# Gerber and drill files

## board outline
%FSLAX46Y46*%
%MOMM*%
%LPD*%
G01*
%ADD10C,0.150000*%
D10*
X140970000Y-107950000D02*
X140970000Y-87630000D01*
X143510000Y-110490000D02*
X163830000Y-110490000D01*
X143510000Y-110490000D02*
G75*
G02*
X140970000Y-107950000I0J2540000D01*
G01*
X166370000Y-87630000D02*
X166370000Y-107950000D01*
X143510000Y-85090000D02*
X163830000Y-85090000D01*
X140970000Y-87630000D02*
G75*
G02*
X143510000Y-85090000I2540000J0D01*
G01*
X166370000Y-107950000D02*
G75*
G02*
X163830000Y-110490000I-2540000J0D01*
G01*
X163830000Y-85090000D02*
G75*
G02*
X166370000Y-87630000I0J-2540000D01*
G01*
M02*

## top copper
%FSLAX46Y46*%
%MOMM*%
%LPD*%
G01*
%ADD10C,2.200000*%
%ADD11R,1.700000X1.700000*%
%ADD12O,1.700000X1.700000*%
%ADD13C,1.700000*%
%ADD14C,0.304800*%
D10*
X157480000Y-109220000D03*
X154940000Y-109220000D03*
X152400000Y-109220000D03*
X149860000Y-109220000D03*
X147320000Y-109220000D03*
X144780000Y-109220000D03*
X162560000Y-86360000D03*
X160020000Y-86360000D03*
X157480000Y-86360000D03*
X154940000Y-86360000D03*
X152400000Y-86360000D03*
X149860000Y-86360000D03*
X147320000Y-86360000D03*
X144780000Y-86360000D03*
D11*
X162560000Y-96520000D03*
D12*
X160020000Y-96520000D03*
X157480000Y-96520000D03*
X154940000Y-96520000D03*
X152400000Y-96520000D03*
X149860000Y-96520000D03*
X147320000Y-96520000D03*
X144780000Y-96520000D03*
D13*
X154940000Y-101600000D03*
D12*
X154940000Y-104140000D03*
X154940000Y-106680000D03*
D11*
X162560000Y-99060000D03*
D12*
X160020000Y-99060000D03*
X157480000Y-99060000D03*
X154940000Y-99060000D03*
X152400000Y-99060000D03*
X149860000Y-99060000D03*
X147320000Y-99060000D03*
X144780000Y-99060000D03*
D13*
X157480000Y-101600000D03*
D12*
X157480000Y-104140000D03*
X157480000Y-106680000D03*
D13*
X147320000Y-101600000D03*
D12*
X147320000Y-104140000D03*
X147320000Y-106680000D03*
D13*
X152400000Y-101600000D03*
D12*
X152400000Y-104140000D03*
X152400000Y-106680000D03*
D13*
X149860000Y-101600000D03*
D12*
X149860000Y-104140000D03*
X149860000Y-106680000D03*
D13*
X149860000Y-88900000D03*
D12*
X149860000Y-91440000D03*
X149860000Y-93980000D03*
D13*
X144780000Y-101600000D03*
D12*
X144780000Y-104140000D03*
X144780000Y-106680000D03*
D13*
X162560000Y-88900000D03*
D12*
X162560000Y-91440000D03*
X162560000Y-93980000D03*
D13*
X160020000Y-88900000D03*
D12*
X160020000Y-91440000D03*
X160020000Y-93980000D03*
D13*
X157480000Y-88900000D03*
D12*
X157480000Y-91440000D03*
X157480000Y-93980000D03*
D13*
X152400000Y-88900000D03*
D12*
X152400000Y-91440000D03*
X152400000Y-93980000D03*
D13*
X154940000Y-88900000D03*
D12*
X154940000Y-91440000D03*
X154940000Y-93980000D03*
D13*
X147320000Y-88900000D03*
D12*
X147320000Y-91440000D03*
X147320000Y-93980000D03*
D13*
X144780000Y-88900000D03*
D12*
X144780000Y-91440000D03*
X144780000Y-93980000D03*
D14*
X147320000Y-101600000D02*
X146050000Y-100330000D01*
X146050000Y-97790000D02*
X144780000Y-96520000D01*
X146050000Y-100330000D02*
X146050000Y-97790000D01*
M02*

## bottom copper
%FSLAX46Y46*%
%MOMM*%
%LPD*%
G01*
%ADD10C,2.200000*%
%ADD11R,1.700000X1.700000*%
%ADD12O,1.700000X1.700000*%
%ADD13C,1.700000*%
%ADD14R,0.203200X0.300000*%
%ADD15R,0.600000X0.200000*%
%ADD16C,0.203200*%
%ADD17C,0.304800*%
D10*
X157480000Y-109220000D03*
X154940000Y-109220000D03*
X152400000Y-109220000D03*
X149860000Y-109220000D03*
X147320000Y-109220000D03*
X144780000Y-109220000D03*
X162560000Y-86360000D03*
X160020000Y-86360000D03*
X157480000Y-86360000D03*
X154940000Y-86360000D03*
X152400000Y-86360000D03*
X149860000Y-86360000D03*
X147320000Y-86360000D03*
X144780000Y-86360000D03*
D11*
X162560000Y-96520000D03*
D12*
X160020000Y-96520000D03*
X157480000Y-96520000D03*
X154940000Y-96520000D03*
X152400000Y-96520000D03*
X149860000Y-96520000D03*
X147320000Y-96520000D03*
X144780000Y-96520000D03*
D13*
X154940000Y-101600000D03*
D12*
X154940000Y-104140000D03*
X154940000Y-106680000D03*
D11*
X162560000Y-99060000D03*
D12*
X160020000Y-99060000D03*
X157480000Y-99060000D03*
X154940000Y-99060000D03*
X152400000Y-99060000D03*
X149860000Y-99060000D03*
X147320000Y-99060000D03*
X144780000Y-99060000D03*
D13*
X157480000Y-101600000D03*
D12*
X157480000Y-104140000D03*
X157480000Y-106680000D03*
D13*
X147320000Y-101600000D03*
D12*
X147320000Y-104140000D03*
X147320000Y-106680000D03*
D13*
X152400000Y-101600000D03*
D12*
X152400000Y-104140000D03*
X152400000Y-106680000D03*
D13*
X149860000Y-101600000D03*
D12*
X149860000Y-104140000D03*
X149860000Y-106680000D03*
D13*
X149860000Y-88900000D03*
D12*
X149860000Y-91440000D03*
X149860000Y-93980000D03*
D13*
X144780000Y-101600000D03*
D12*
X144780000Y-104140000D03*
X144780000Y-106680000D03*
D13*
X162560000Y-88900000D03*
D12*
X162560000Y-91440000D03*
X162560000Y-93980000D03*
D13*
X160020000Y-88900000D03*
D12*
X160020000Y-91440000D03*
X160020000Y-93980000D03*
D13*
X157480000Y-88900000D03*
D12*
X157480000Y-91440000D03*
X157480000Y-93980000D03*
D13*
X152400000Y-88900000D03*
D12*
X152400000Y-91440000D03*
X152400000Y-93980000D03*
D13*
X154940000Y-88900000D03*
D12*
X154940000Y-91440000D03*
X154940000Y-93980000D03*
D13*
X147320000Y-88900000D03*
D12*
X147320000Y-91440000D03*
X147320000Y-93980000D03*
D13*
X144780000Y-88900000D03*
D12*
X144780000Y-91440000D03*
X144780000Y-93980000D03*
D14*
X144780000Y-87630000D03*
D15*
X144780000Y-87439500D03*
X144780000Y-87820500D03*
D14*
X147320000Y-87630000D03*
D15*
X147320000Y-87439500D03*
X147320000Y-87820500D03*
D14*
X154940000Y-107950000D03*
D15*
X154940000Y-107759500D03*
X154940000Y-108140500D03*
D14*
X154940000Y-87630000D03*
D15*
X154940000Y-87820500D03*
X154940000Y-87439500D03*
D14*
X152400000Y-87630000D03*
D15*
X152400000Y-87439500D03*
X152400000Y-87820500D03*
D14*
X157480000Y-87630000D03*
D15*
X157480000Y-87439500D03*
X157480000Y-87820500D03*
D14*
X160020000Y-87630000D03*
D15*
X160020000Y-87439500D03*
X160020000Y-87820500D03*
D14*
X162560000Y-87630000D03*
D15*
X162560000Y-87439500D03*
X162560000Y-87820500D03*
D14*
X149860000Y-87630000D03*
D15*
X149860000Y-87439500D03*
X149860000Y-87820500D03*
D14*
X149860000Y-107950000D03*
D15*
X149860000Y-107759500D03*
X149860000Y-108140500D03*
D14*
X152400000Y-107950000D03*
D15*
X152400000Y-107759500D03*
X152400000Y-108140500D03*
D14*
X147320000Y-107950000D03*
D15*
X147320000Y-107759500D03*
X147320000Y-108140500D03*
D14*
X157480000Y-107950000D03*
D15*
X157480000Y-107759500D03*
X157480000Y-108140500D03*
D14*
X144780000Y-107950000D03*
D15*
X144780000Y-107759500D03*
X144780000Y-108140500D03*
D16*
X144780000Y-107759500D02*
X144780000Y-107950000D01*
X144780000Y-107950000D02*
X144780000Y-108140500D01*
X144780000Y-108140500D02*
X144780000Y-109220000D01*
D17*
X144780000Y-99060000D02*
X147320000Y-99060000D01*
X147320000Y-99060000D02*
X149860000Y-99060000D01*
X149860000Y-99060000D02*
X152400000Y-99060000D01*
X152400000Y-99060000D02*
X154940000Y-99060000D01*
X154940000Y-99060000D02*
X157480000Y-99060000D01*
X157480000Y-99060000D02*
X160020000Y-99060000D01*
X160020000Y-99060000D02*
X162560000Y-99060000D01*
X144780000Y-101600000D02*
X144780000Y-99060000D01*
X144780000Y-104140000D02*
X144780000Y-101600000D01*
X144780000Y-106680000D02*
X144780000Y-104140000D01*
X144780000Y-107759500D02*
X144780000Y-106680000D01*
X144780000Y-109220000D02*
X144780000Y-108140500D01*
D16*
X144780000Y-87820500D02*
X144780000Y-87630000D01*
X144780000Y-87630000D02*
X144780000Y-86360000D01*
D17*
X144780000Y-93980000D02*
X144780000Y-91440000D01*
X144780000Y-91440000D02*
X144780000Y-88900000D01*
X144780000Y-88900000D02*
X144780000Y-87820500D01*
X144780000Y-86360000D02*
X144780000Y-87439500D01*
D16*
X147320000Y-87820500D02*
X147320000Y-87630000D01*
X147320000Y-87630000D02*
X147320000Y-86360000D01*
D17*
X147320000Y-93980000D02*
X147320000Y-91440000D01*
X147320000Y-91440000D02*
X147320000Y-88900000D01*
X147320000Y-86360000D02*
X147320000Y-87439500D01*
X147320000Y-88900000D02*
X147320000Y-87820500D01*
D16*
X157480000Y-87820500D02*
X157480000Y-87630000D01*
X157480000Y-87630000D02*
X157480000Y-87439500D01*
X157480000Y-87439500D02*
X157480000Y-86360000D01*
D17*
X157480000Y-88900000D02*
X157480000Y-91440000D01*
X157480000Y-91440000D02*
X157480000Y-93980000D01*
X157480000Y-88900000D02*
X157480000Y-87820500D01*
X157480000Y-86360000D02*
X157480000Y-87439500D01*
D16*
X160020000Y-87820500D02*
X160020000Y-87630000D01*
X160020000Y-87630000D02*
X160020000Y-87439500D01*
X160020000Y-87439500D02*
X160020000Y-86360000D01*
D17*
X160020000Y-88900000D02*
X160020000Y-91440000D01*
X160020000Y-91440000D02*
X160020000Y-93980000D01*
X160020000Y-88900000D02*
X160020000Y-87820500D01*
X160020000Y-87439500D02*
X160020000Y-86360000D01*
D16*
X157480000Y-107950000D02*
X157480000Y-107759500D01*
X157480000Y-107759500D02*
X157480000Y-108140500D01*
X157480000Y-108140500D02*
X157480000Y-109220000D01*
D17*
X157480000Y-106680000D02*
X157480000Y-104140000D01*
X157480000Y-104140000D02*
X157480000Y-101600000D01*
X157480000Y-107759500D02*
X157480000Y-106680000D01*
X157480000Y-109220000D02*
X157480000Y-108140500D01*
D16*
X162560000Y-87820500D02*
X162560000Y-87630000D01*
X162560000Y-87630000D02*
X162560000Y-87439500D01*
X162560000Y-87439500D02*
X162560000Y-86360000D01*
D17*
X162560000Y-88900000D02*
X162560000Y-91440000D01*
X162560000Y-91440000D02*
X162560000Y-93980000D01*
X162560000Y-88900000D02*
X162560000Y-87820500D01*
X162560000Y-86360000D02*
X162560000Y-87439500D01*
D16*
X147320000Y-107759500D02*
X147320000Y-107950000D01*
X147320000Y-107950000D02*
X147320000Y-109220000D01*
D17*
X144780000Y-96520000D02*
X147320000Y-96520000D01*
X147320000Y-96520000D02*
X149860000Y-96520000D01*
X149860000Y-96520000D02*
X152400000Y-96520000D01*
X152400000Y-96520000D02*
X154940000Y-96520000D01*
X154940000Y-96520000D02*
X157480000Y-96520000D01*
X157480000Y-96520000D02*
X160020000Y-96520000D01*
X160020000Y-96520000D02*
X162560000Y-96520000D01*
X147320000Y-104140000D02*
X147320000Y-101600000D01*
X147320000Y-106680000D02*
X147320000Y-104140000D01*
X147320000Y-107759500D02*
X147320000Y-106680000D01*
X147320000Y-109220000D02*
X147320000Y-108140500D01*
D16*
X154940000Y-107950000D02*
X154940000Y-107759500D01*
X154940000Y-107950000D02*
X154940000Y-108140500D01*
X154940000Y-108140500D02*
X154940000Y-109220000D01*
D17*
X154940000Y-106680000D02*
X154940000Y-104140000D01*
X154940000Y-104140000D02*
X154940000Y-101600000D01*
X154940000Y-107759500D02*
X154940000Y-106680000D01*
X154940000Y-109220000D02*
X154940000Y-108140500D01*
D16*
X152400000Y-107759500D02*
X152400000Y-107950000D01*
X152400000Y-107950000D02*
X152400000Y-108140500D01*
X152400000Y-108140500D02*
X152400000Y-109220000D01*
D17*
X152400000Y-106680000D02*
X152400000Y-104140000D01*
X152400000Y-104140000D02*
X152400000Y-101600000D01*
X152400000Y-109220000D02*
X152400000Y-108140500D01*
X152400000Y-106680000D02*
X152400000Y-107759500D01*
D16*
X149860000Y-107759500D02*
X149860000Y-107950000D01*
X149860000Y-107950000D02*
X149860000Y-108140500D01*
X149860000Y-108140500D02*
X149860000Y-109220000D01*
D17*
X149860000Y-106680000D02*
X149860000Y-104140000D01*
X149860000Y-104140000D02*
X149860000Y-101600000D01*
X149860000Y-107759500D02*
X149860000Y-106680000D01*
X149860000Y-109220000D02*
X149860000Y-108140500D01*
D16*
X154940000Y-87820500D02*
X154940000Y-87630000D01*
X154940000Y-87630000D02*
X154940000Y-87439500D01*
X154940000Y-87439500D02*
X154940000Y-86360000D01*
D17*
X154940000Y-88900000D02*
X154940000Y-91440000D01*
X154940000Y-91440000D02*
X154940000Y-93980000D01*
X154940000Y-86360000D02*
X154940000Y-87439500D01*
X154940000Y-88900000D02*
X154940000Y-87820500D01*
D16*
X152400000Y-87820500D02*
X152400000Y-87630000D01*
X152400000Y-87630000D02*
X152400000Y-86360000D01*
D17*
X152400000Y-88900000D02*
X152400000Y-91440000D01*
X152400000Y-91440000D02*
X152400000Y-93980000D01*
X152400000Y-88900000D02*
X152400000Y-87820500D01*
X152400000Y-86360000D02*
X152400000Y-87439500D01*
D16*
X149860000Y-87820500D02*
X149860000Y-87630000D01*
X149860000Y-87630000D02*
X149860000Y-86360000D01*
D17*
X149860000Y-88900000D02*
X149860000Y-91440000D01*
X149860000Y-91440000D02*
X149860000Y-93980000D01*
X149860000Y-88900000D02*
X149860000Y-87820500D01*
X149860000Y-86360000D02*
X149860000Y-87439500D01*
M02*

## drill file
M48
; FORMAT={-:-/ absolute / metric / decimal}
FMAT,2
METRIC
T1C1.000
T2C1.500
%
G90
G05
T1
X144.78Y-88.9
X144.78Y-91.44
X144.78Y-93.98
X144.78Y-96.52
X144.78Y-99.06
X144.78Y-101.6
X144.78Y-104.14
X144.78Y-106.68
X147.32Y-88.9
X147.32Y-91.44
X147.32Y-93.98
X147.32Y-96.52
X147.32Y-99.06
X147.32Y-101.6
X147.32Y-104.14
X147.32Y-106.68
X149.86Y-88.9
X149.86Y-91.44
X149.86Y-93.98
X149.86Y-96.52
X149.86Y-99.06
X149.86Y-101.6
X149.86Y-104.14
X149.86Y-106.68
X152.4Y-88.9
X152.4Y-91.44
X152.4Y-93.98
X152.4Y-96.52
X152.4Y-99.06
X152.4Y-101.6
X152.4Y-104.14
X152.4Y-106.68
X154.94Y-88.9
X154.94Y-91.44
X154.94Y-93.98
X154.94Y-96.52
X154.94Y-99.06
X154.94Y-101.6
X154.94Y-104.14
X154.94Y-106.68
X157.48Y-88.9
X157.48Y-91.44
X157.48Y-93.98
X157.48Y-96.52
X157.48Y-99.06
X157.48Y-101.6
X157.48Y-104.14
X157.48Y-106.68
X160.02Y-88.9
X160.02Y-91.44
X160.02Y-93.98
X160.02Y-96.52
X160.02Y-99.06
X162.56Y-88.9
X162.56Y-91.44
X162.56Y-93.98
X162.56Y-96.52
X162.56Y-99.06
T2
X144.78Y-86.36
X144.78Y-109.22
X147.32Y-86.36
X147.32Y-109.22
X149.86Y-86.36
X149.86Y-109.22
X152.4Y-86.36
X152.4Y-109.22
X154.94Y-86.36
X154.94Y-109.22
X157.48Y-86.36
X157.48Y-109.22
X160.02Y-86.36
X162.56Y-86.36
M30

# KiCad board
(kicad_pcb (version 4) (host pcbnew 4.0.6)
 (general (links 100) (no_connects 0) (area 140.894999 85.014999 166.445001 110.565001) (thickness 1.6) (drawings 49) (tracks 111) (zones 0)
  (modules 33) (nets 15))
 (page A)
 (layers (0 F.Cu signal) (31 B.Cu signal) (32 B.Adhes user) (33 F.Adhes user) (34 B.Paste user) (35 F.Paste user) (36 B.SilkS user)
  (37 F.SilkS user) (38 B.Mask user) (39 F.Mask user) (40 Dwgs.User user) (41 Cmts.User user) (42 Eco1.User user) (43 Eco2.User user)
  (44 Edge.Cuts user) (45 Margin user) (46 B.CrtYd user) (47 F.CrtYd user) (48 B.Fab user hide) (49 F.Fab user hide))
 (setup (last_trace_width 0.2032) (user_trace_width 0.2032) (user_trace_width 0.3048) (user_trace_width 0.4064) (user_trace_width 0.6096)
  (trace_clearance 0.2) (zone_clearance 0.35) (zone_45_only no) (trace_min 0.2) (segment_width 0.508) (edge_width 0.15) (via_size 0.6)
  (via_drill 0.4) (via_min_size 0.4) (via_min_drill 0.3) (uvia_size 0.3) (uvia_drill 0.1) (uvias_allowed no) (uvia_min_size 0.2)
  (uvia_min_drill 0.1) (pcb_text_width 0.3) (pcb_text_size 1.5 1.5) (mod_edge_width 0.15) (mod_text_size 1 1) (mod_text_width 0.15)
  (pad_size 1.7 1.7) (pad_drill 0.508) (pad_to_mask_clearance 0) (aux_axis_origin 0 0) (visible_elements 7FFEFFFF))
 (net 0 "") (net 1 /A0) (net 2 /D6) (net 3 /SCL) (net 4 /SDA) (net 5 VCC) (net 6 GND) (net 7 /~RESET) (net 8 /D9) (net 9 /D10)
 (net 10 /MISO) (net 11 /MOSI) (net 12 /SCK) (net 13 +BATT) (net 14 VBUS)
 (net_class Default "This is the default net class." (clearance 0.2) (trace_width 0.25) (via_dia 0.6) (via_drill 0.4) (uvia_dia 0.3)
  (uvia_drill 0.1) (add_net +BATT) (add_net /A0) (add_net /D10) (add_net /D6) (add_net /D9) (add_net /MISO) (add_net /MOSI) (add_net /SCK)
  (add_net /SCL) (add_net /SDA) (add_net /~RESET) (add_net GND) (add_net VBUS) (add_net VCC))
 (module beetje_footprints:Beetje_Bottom (layer F.Cu) (at 157.48 109.22 270)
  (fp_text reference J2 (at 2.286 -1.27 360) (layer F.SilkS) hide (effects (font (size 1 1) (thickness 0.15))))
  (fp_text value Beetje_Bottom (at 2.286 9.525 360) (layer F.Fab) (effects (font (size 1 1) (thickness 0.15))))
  (pad 1 thru_hole circle (at 0 0 270) (size 2.2 2.2) (drill 1.5) (layers *.Cu *.Mask) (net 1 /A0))
  (pad 2 thru_hole circle (at 0 2.54 270) (size 2.2 2.2) (drill 1.5) (layers *.Cu *.Mask) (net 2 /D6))
  (pad 3 thru_hole circle (at 0 5.08 270) (size 2.2 2.2) (drill 1.5) (layers *.Cu *.Mask) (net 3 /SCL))
  (pad 4 thru_hole circle (at 0 7.62 270) (size 2.2 2.2) (drill 1.5) (layers *.Cu *.Mask) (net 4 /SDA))
  (pad 5 thru_hole circle (at 0 10.16 270) (size 2.2 2.2) (drill 1.5) (layers *.Cu *.Mask) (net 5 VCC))
  (pad 6 thru_hole circle (at 0 12.7 270) (size 2.2 2.2) (drill 1.5) (layers *.Cu *.Mask) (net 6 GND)))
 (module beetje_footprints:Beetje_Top (layer F.Cu) (at 162.56 86.36 270)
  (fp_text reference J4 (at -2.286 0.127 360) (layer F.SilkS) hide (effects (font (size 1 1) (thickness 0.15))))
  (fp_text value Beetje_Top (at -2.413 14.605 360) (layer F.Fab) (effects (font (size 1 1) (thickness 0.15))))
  (pad 1 thru_hole circle (at 0 0 270) (size 2.2 2.2) (drill 1.5) (layers *.Cu *.Mask) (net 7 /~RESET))
  (pad 2 thru_hole circle (at 0 2.54 270) (size 2.2 2.2) (drill 1.5) (layers *.Cu *.Mask) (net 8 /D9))
  (pad 3 thru_hole circle (at 0 5.08 270) (size 2.2 2.2) (drill 1.5) (layers *.Cu *.Mask) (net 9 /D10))
  (pad 4 thru_hole circle (at 0 7.62 270) (size 2.2 2.2) (drill 1.5) (layers *.Cu *.Mask) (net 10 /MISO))
  (pad 5 thru_hole circle (at 0 10.16 270) (size 2.2 2.2) (drill 1.5) (layers *.Cu *.Mask) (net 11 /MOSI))
  (pad 6 thru_hole circle (at 0 12.7 270) (size 2.2 2.2) (drill 1.5) (layers *.Cu *.Mask) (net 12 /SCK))
  (pad 7 thru_hole circle (at 0 15.24 270) (size 2.2 2.2) (drill 1.5) (layers *.Cu *.Mask) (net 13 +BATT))
  (pad 8 thru_hole circle (at 0 17.78 270) (size 2.2 2.2) (drill 1.5) (layers *.Cu *.Mask) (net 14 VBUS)))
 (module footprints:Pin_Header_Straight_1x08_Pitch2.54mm (layer F.Cu) (at 162.56 96.52 270)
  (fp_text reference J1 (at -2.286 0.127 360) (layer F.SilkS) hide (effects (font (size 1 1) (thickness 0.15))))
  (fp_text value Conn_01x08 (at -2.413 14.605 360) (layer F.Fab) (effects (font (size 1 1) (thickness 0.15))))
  (pad 1 thru_hole rect (at 0 0 270) (size 1.7 1.7) (drill 1) (layers *.Cu *.Mask) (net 5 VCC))
  (pad 2 thru_hole oval (at 0 2.54 270) (size 1.7 1.7) (drill 1) (layers *.Cu *.Mask) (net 5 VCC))
  (pad 3 thru_hole oval (at 0 5.08 270) (size 1.7 1.7) (drill 1) (layers *.Cu *.Mask) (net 5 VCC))
  (pad 4 thru_hole oval (at 0 7.62 270) (size 1.7 1.7) (drill 1) (layers *.Cu *.Mask) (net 5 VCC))
  (pad 5 thru_hole oval (at 0 10.16 270) (size 1.7 1.7) (drill 1) (layers *.Cu *.Mask) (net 5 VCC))
  (pad 6 thru_hole oval (at 0 12.7 270) (size 1.7 1.7) (drill 1) (layers *.Cu *.Mask) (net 5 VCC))
  (pad 7 thru_hole oval (at 0 15.24 270) (size 1.7 1.7) (drill 1) (layers *.Cu *.Mask) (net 5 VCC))
  (pad 8 thru_hole oval (at 0 17.78 270) (size 1.7 1.7) (drill 1) (layers *.Cu *.Mask) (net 5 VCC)))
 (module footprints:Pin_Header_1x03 (layer F.Cu) (at 154.94 101.6)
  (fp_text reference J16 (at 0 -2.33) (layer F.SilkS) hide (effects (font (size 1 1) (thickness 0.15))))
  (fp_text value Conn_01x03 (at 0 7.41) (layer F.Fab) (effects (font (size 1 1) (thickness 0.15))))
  (pad 1 thru_hole circle (at 0 0) (size 1.7 1.7) (drill 1) (layers *.Cu *.Mask) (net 2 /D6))
  (pad 2 thru_hole oval (at 0 2.54) (size 1.7 1.7) (drill 1) (layers *.Cu *.Mask) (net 2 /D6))
  (pad 3 thru_hole oval (at 0 5.08) (size 1.7 1.7) (drill 1) (layers *.Cu *.Mask) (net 2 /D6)))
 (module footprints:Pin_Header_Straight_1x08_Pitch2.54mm (layer F.Cu) (at 162.56 99.06 270)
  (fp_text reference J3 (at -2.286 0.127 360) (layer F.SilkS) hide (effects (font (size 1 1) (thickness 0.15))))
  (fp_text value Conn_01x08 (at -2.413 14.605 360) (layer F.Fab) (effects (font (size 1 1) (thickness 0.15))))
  (pad 1 thru_hole rect (at 0 0 270) (size 1.7 1.7) (drill 1) (layers *.Cu *.Mask) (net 6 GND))
  (pad 2 thru_hole oval (at 0 2.54 270) (size 1.7 1.7) (drill 1) (layers *.Cu *.Mask) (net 6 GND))
  (pad 3 thru_hole oval (at 0 5.08 270) (size 1.7 1.7) (drill 1) (layers *.Cu *.Mask) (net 6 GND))
  (pad 4 thru_hole oval (at 0 7.62 270) (size 1.7 1.7) (drill 1) (layers *.Cu *.Mask) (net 6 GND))
  (pad 5 thru_hole oval (at 0 10.16 270) (size 1.7 1.7) (drill 1) (layers *.Cu *.Mask) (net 6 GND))
  (pad 6 thru_hole oval (at 0 12.7 270) (size 1.7 1.7) (drill 1) (layers *.Cu *.Mask) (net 6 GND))
  (pad 7 thru_hole oval (at 0 15.24 270) (size 1.7 1.7) (drill 1) (layers *.Cu *.Mask) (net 6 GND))
  (pad 8 thru_hole oval (at 0 17.78 270) (size 1.7 1.7) (drill 1) (layers *.Cu *.Mask) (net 6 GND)))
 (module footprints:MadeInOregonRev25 (layer F.Cu) (at 162.56 102.87)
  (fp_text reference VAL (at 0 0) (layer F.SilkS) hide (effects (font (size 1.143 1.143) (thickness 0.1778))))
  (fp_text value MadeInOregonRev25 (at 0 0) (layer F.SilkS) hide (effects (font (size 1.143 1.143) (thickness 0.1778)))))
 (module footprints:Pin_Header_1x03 (layer F.Cu) (at 157.48 101.6)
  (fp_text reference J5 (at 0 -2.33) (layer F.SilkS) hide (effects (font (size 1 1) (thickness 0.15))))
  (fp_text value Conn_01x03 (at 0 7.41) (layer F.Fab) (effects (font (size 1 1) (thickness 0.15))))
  (pad 1 thru_hole circle (at 0 0) (size 1.7 1.7) (drill 1) (layers *.Cu *.Mask) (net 1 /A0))
  (pad 2 thru_hole oval (at 0 2.54) (size 1.7 1.7) (drill 1) (layers *.Cu *.Mask) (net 1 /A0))
  (pad 3 thru_hole oval (at 0 5.08) (size 1.7 1.7) (drill 1) (layers *.Cu *.Mask) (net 1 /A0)))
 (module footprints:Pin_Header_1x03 (layer F.Cu) (at 147.32 101.6)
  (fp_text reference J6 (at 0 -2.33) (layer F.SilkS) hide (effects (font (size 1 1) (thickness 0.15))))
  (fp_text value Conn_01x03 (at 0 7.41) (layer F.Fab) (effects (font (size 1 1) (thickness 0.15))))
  (pad 1 thru_hole circle (at 0 0) (size 1.7 1.7) (drill 1) (layers *.Cu *.Mask) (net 5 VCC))
  (pad 2 thru_hole oval (at 0 2.54) (size 1.7 1.7) (drill 1) (layers *.Cu *.Mask) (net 5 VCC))
  (pad 3 thru_hole oval (at 0 5.08) (size 1.7 1.7) (drill 1) (layers *.Cu *.Mask) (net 5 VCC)))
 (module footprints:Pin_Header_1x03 (layer F.Cu) (at 152.4 101.6)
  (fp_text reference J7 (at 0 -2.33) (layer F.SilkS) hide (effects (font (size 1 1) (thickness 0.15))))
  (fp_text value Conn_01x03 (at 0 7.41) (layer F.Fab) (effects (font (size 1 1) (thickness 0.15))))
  (pad 1 thru_hole circle (at 0 0) (size 1.7 1.7) (drill 1) (layers *.Cu *.Mask) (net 3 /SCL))
  (pad 2 thru_hole oval (at 0 2.54) (size 1.7 1.7) (drill 1) (layers *.Cu *.Mask) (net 3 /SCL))
  (pad 3 thru_hole oval (at 0 5.08) (size 1.7 1.7) (drill 1) (layers *.Cu *.Mask) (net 3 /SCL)))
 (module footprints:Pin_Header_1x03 (layer F.Cu) (at 149.86 101.6)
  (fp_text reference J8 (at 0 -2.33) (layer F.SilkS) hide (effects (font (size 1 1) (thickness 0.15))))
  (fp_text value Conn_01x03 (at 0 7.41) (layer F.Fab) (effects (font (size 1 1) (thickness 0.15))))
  (pad 1 thru_hole circle (at 0 0) (size 1.7 1.7) (drill 1) (layers *.Cu *.Mask) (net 4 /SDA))
  (pad 2 thru_hole oval (at 0 2.54) (size 1.7 1.7) (drill 1) (layers *.Cu *.Mask) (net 4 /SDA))
  (pad 3 thru_hole oval (at 0 5.08) (size 1.7 1.7) (drill 1) (layers *.Cu *.Mask) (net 4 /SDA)))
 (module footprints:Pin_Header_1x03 (layer F.Cu) (at 149.86 88.9)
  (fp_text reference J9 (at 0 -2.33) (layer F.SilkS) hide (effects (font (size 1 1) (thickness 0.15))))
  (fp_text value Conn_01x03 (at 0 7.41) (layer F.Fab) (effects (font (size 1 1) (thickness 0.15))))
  (pad 1 thru_hole circle (at 0 0) (size 1.7 1.7) (drill 1) (layers *.Cu *.Mask) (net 12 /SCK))
  (pad 2 thru_hole oval (at 0 2.54) (size 1.7 1.7) (drill 1) (layers *.Cu *.Mask) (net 12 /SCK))
  (pad 3 thru_hole oval (at 0 5.08) (size 1.7 1.7) (drill 1) (layers *.Cu *.Mask) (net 12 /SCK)))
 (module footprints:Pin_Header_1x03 (layer F.Cu) (at 144.78 101.6)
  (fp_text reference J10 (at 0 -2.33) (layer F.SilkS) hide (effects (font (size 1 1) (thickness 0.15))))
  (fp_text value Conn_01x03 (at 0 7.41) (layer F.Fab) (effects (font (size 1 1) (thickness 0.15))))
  (pad 1 thru_hole circle (at 0 0) (size 1.7 1.7) (drill 1) (layers *.Cu *.Mask) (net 6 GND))
  (pad 2 thru_hole oval (at 0 2.54) (size 1.7 1.7) (drill 1) (layers *.Cu *.Mask) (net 6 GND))
  (pad 3 thru_hole oval (at 0 5.08) (size 1.7 1.7) (drill 1) (layers *.Cu *.Mask) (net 6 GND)))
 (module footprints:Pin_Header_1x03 (layer F.Cu) (at 162.56 88.9)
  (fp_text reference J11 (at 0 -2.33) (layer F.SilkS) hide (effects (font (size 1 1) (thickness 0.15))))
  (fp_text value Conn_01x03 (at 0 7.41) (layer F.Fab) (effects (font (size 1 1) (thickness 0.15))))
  (pad 1 thru_hole circle (at 0 0) (size 1.7 1.7) (drill 1) (layers *.Cu *.Mask) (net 7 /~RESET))
  (pad 2 thru_hole oval (at 0 2.54) (size 1.7 1.7) (drill 1) (layers *.Cu *.Mask) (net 7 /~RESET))
  (pad 3 thru_hole oval (at 0 5.08) (size 1.7 1.7) (drill 1) (layers *.Cu *.Mask) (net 7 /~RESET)))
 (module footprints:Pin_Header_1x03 (layer F.Cu) (at 160.02 88.9)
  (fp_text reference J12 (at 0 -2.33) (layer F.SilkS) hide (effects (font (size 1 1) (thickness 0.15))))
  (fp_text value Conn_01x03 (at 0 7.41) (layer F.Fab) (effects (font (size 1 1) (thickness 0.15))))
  (pad 1 thru_hole circle (at 0 0) (size 1.7 1.7) (drill 1) (layers *.Cu *.Mask) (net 8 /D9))
  (pad 2 thru_hole oval (at 0 2.54) (size 1.7 1.7) (drill 1) (layers *.Cu *.Mask) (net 8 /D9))
  (pad 3 thru_hole oval (at 0 5.08) (size 1.7 1.7) (drill 1) (layers *.Cu *.Mask) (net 8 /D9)))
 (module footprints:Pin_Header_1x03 (layer F.Cu) (at 157.48 88.9)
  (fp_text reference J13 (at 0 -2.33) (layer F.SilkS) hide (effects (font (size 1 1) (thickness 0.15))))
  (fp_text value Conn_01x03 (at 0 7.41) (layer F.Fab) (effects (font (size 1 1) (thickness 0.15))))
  (pad 1 thru_hole circle (at 0 0) (size 1.7 1.7) (drill 1) (layers *.Cu *.Mask) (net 9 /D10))
  (pad 2 thru_hole oval (at 0 2.54) (size 1.7 1.7) (drill 1) (layers *.Cu *.Mask) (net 9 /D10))
  (pad 3 thru_hole oval (at 0 5.08) (size 1.7 1.7) (drill 1) (layers *.Cu *.Mask) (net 9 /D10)))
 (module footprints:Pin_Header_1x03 (layer F.Cu) (at 152.4 88.9)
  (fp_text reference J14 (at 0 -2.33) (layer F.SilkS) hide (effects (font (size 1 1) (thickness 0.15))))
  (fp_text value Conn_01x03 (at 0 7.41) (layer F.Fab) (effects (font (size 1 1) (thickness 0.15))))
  (pad 1 thru_hole circle (at 0 0) (size 1.7 1.7) (drill 1) (layers *.Cu *.Mask) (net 11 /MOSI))
  (pad 2 thru_hole oval (at 0 2.54) (size 1.7 1.7) (drill 1) (layers *.Cu *.Mask) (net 11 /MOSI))
  (pad 3 thru_hole oval (at 0 5.08) (size 1.7 1.7) (drill 1) (layers *.Cu *.Mask) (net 11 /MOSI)))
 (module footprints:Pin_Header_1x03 (layer F.Cu) (at 154.94 88.9)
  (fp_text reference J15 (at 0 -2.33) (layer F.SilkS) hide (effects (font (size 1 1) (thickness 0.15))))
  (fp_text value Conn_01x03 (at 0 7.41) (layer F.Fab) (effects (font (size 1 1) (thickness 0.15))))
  (pad 1 thru_hole circle (at 0 0) (size 1.7 1.7) (drill 1) (layers *.Cu *.Mask) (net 10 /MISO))
  (pad 2 thru_hole oval (at 0 2.54) (size 1.7 1.7) (drill 1) (layers *.Cu *.Mask) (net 10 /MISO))
  (pad 3 thru_hole oval (at 0 5.08) (size 1.7 1.7) (drill 1) (layers *.Cu *.Mask) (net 10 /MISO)))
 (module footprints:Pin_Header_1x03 (layer F.Cu) (at 147.32 88.9)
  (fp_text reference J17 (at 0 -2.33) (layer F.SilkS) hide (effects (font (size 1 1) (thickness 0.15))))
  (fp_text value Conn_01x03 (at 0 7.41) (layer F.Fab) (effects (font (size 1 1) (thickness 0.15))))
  (pad 1 thru_hole circle (at 0 0) (size 1.7 1.7) (drill 1) (layers *.Cu *.Mask) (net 13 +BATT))
  (pad 2 thru_hole oval (at 0 2.54) (size 1.7 1.7) (drill 1) (layers *.Cu *.Mask) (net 13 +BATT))
  (pad 3 thru_hole oval (at 0 5.08) (size 1.7 1.7) (drill 1) (layers *.Cu *.Mask) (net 13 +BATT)))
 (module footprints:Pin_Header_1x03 (layer F.Cu) (at 144.78 88.9)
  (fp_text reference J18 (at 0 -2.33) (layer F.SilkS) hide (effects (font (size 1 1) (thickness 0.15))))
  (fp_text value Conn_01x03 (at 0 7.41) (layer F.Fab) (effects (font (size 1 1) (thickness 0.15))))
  (pad 1 thru_hole circle (at 0 0) (size 1.7 1.7) (drill 1) (layers *.Cu *.Mask) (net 14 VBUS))
  (pad 2 thru_hole oval (at 0 2.54) (size 1.7 1.7) (drill 1) (layers *.Cu *.Mask) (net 14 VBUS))
  (pad 3 thru_hole oval (at 0 5.08) (size 1.7 1.7) (drill 1) (layers *.Cu *.Mask) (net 14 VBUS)))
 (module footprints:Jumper (layer B.Cu) (at 144.78 87.63 270)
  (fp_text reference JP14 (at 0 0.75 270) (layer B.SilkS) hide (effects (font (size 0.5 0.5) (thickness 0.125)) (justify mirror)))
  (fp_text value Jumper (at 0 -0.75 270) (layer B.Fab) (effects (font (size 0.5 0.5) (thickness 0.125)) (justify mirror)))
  (pad 1 smd rect (at 0 0 270) (size 0.3 0.2032) (layers B.Cu B.Paste B.Mask) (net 14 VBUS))
  (pad 1 smd rect (at -0.1905 0 270) (size 0.2 0.6) (layers B.Cu) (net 14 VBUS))
  (pad 1 smd rect (at 0.1905 0 270) (size 0.2 0.6) (layers B.Cu) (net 14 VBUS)))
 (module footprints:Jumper (layer B.Cu) (at 147.32 87.63 270)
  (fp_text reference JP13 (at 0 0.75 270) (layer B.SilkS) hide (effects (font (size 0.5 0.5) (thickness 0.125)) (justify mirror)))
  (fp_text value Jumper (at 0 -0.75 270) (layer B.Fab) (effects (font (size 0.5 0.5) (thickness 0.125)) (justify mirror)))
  (pad 1 smd rect (at 0 0 270) (size 0.3 0.2032) (layers B.Cu B.Paste B.Mask) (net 13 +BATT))
  (pad 1 smd rect (at -0.1905 0 270) (size 0.2 0.6) (layers B.Cu) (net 13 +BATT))
  (pad 1 smd rect (at 0.1905 0 270) (size 0.2 0.6) (layers B.Cu) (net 13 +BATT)))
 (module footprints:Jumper (layer B.Cu) (at 154.94 107.95 270)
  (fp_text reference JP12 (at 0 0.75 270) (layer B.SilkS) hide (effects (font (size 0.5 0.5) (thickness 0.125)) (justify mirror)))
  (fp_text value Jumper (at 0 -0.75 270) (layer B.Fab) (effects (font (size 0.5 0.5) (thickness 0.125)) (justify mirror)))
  (pad 1 smd rect (at 0 0 270) (size 0.3 0.2032) (layers B.Cu B.Paste B.Mask) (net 2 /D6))
  (pad 1 smd rect (at -0.1905 0 270) (size 0.2 0.6) (layers B.Cu) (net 2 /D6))
  (pad 1 smd rect (at 0.1905 0 270) (size 0.2 0.6) (layers B.Cu) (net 2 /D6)))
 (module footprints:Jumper (layer B.Cu) (at 154.94 87.63 90)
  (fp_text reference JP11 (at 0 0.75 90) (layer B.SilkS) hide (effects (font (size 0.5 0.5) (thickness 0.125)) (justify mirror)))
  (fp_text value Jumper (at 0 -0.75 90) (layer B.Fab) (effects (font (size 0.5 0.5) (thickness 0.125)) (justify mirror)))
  (pad 1 smd rect (at 0 0 90) (size 0.3 0.2032) (layers B.Cu B.Paste B.Mask) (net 10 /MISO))
  (pad 1 smd rect (at -0.1905 0 90) (size 0.2 0.6) (layers B.Cu) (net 10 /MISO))
  (pad 1 smd rect (at 0.1905 0 90) (size 0.2 0.6) (layers B.Cu) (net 10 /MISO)))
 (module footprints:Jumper (layer B.Cu) (at 152.4 87.63 270)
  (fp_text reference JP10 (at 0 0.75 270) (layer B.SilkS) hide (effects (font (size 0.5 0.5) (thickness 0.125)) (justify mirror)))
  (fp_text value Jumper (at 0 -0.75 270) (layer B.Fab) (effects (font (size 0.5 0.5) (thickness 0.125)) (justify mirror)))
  (pad 1 smd rect (at 0 0 270) (size 0.3 0.2032) (layers B.Cu B.Paste B.Mask) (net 11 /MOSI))
  (pad 1 smd rect (at -0.1905 0 270) (size 0.2 0.6) (layers B.Cu) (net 11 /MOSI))
  (pad 1 smd rect (at 0.1905 0 270) (size 0.2 0.6) (layers B.Cu) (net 11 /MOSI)))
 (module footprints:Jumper (layer B.Cu) (at 157.48 87.63 270)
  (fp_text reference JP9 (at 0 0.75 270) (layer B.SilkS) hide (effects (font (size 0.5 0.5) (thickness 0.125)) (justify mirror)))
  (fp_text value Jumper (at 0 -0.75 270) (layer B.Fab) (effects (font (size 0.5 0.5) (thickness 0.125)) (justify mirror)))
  (pad 1 smd rect (at 0 0 270) (size 0.3 0.2032) (layers B.Cu B.Paste B.Mask) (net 9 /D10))
  (pad 1 smd rect (at -0.1905 0 270) (size 0.2 0.6) (layers B.Cu) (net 9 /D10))
  (pad 1 smd rect (at 0.1905 0 270) (size 0.2 0.6) (layers B.Cu) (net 9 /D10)))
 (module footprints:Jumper (layer B.Cu) (at 160.02 87.63 270)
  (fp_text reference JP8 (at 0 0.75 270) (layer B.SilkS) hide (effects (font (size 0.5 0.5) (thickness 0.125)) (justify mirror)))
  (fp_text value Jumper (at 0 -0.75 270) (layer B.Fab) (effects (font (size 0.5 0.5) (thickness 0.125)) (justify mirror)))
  (pad 1 smd rect (at 0 0 270) (size 0.3 0.2032) (layers B.Cu B.Paste B.Mask) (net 8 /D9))
  (pad 1 smd rect (at -0.1905 0 270) (size 0.2 0.6) (layers B.Cu) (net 8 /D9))
  (pad 1 smd rect (at 0.1905 0 270) (size 0.2 0.6) (layers B.Cu) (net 8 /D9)))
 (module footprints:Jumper (layer B.Cu) (at 162.56 87.63 270)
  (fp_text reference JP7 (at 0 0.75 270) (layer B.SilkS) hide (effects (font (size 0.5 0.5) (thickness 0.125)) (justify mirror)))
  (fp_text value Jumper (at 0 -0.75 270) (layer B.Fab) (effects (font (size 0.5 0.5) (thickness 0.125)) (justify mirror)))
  (pad 1 smd rect (at 0 0 270) (size 0.3 0.2032) (layers B.Cu B.Paste B.Mask) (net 7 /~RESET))
  (pad 1 smd rect (at -0.1905 0 270) (size 0.2 0.6) (layers B.Cu) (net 7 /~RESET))
  (pad 1 smd rect (at 0.1905 0 270) (size 0.2 0.6) (layers B.Cu) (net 7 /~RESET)))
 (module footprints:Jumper (layer B.Cu) (at 149.86 87.63 270)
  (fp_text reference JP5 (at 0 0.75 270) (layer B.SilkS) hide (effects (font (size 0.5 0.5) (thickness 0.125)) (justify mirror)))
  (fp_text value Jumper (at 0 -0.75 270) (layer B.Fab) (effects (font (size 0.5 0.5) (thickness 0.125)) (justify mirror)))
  (pad 1 smd rect (at 0 0 270) (size 0.3 0.2032) (layers B.Cu B.Paste B.Mask) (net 12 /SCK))
  (pad 1 smd rect (at -0.1905 0 270) (size 0.2 0.6) (layers B.Cu) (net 12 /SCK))
  (pad 1 smd rect (at 0.1905 0 270) (size 0.2 0.6) (layers B.Cu) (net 12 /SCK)))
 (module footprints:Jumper (layer B.Cu) (at 149.86 107.95 270)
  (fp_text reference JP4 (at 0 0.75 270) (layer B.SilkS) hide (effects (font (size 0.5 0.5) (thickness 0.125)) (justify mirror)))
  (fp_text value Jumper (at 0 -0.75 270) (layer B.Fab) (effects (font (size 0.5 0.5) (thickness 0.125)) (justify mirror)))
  (pad 1 smd rect (at 0 0 270) (size 0.3 0.2032) (layers B.Cu B.Paste B.Mask) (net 4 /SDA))
  (pad 1 smd rect (at -0.1905 0 270) (size 0.2 0.6) (layers B.Cu) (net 4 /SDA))
  (pad 1 smd rect (at 0.1905 0 270) (size 0.2 0.6) (layers B.Cu) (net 4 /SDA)))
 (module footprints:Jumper (layer B.Cu) (at 152.4 107.95 270)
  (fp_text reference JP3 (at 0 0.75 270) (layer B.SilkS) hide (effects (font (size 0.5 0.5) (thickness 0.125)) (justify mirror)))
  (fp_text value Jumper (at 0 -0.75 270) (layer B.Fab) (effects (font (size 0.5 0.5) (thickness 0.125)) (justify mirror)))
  (pad 1 smd rect (at 0 0 270) (size 0.3 0.2032) (layers B.Cu B.Paste B.Mask) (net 3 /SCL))
  (pad 1 smd rect (at -0.1905 0 270) (size 0.2 0.6) (layers B.Cu) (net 3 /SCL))
  (pad 1 smd rect (at 0.1905 0 270) (size 0.2 0.6) (layers B.Cu) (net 3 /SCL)))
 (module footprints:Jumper (layer B.Cu) (at 147.32 107.95 270)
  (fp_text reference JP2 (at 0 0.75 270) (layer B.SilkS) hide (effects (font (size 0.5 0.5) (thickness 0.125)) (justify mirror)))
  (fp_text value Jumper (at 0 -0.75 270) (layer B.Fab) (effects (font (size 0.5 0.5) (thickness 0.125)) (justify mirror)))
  (pad 1 smd rect (at 0 0 270) (size 0.3 0.2032) (layers B.Cu B.Paste B.Mask) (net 5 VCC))
  (pad 1 smd rect (at -0.1905 0 270) (size 0.2 0.6) (layers B.Cu) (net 5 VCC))
  (pad 1 smd rect (at 0.1905 0 270) (size 0.2 0.6) (layers B.Cu) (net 5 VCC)))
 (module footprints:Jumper (layer B.Cu) (at 157.48 107.95 270)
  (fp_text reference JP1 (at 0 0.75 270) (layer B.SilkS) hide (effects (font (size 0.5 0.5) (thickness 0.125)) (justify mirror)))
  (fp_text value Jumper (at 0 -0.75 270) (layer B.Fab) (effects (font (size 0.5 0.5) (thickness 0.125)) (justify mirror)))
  (pad 1 smd rect (at 0 0 270) (size 0.3 0.2032) (layers B.Cu B.Paste B.Mask) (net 1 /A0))
  (pad 1 smd rect (at -0.1905 0 270) (size 0.2 0.6) (layers B.Cu) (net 1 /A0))
  (pad 1 smd rect (at 0.1905 0 270) (size 0.2 0.6) (layers B.Cu) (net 1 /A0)))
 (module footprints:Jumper (layer B.Cu) (at 144.78 107.95 270)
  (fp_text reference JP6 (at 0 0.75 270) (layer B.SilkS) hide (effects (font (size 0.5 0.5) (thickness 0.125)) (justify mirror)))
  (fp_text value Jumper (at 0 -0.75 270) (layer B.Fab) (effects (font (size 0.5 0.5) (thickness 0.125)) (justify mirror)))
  (pad 1 smd rect (at 0 0 270) (size 0.3 0.2032) (layers B.Cu B.Paste B.Mask) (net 6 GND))
  (pad 1 smd rect (at -0.1905 0 270) (size 0.2 0.6) (layers B.Cu) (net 6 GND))
  (pad 1 smd rect (at 0.1905 0 270) (size 0.2 0.6) (layers B.Cu) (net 6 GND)))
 (gr_line (start 140.97 107.95) (end 140.97 87.63) (angle 90) (layer Edge.Cuts) (width 0.15))
 (gr_line (start 143.51 110.49) (end 163.83 110.49) (angle 90) (layer Edge.Cuts) (width 0.15))
 (gr_arc (start 143.51 107.95) (end 143.51 110.49) (angle 90) (layer Edge.Cuts) (width 0.15))
 (gr_line (start 166.37 87.63) (end 166.37 107.95) (angle 90) (layer Edge.Cuts) (width 0.15))
 (gr_line (start 143.51 85.09) (end 163.83 85.09) (angle 90) (layer Edge.Cuts) (width 0.15))
 (gr_arc (start 143.51 87.63) (end 140.97 87.63) (angle 90) (layer Edge.Cuts) (width 0.15))
 (gr_arc (start 163.83 107.95) (end 166.37 107.95) (angle 90) (layer Edge.Cuts) (width 0.15))
 (gr_arc (start 163.83 87.63) (end 163.83 85.09) (angle 90) (layer Edge.Cuts) (width 0.15))
 (segment (start 144.78 107.7595) (end 144.78 107.95) (width 0.2032) (layer B.Cu) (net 6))
 (segment (start 144.78 107.95) (end 144.78 108.1405) (width 0.2032) (layer B.Cu) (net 6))
 (segment (start 144.78 108.1405) (end 144.78 109.22) (width 0.2032) (layer B.Cu) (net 6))
 (segment (start 144.78 99.06) (end 147.32 99.06) (width 0.3048) (layer B.Cu) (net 6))
 (segment (start 147.32 99.06) (end 149.86 99.06) (width 0.3048) (layer B.Cu) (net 6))
 (segment (start 149.86 99.06) (end 152.4 99.06) (width 0.3048) (layer B.Cu) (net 6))
 (segment (start 152.4 99.06) (end 154.94 99.06) (width 0.3048) (layer B.Cu) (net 6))
 (segment (start 154.94 99.06) (end 157.48 99.06) (width 0.3048) (layer B.Cu) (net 6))
 (segment (start 157.48 99.06) (end 160.02 99.06) (width 0.3048) (layer B.Cu) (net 6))
 (segment (start 160.02 99.06) (end 162.56 99.06) (width 0.3048) (layer B.Cu) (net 6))
 (segment (start 144.78 101.6) (end 144.78 99.06) (width 0.3048) (layer B.Cu) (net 6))
 (segment (start 144.78 104.14) (end 144.78 101.6) (width 0.3048) (layer B.Cu) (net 6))
 (segment (start 144.78 106.68) (end 144.78 104.14) (width 0.3048) (layer B.Cu) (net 6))
 (segment (start 144.78 107.7595) (end 144.78 106.68) (width 0.3048) (layer B.Cu) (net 6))
 (segment (start 144.78 109.22) (end 144.78 108.1405) (width 0.3048) (layer B.Cu) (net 6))
 (segment (start 144.78 87.8205) (end 144.78 87.63) (width 0.2032) (layer B.Cu) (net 14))
 (segment (start 144.78 87.63) (end 144.78 86.36) (width 0.2032) (layer B.Cu) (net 14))
 (segment (start 144.78 93.98) (end 144.78 91.44) (width 0.3048) (layer B.Cu) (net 14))
 (segment (start 144.78 91.44) (end 144.78 88.9) (width 0.3048) (layer B.Cu) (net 14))
 (segment (start 144.78 88.9) (end 144.78 87.8205) (width 0.3048) (layer B.Cu) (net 14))
 (segment (start 144.78 86.36) (end 144.78 87.4395) (width 0.3048) (layer B.Cu) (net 14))
 (segment (start 147.32 87.8205) (end 147.32 87.63) (width 0.2032) (layer B.Cu) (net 13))
 (segment (start 147.32 87.63) (end 147.32 86.36) (width 0.2032) (layer B.Cu) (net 13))
 (segment (start 147.32 93.98) (end 147.32 91.44) (width 0.3048) (layer B.Cu) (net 13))
 (segment (start 147.32 91.44) (end 147.32 88.9) (width 0.3048) (layer B.Cu) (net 13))
 (segment (start 147.32 86.36) (end 147.32 87.4395) (width 0.3048) (layer B.Cu) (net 13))
 (segment (start 147.32 88.9) (end 147.32 87.8205) (width 0.3048) (layer B.Cu) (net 13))
 (segment (start 157.48 87.8205) (end 157.48 87.63) (width 0.2032) (layer B.Cu) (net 9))
 (segment (start 157.48 87.63) (end 157.48 87.4395) (width 0.2032) (layer B.Cu) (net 9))
 (segment (start 157.48 87.4395) (end 157.48 86.36) (width 0.2032) (layer B.Cu) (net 9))
 (segment (start 157.48 88.9) (end 157.48 91.44) (width 0.3048) (layer B.Cu) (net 9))
 (segment (start 157.48 91.44) (end 157.48 93.98) (width 0.3048) (layer B.Cu) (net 9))
 (segment (start 157.48 88.9) (end 157.48 87.8205) (width 0.3048) (layer B.Cu) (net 9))
 (segment (start 157.48 86.36) (end 157.48 87.4395) (width 0.3048) (layer B.Cu) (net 9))
 (segment (start 160.02 87.8205) (end 160.02 87.63) (width 0.2032) (layer B.Cu) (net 8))
 (segment (start 160.02 87.63) (end 160.02 87.4395) (width 0.2032) (layer B.Cu) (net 8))
 (segment (start 160.02 87.4395) (end 160.02 86.36) (width 0.2032) (layer B.Cu) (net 8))
 (segment (start 160.02 88.9) (end 160.02 91.44) (width 0.3048) (layer B.Cu) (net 8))
 (segment (start 160.02 91.44) (end 160.02 93.98) (width 0.3048) (layer B.Cu) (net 8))
 (segment (start 160.02 88.9) (end 160.02 87.8205) (width 0.3048) (layer B.Cu) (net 8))
 (segment (start 160.02 87.4395) (end 160.02 86.36) (width 0.3048) (layer B.Cu) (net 8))
 (segment (start 157.48 107.95) (end 157.48 107.7595) (width 0.2032) (layer B.Cu) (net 1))
 (segment (start 157.48 107.7595) (end 157.48 108.1405) (width 0.2032) (layer B.Cu) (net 1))
 (segment (start 157.48 108.1405) (end 157.48 109.22) (width 0.2032) (layer B.Cu) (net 1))
 (segment (start 157.48 106.68) (end 157.48 104.14) (width 0.3048) (layer B.Cu) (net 1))
 (segment (start 157.48 104.14) (end 157.48 101.6) (width 0.3048) (layer B.Cu) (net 1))
 (segment (start 157.48 107.7595) (end 157.48 106.68) (width 0.3048) (layer B.Cu) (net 1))
 (segment (start 157.48 109.22) (end 157.48 108.1405) (width 0.3048) (layer B.Cu) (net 1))
 (segment (start 162.56 87.8205) (end 162.56 87.63) (width 0.2032) (layer B.Cu) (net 7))
 (segment (start 162.56 87.63) (end 162.56 87.4395) (width 0.2032) (layer B.Cu) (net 7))
 (segment (start 162.56 87.4395) (end 162.56 86.36) (width 0.2032) (layer B.Cu) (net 7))
 (segment (start 162.56 88.9) (end 162.56 91.44) (width 0.3048) (layer B.Cu) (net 7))
 (segment (start 162.56 91.44) (end 162.56 93.98) (width 0.3048) (layer B.Cu) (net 7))
 (segment (start 162.56 88.9) (end 162.56 87.8205) (width 0.3048) (layer B.Cu) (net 7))
 (segment (start 162.56 86.36) (end 162.56 87.4395) (width 0.3048) (layer B.Cu) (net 7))
 (segment (start 147.32 107.7595) (end 147.32 107.95) (width 0.2032) (layer B.Cu) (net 5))
 (segment (start 147.32 107.95) (end 147.32 109.22) (width 0.2032) (layer B.Cu) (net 5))
 (segment (start 147.32 101.6) (end 146.05 100.33) (width 0.3048) (layer F.Cu) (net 5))
 (segment (start 146.05 97.79) (end 144.78 96.52) (width 0.3048) (layer F.Cu) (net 5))
 (segment (start 146.05 100.33) (end 146.05 97.79) (width 0.3048) (layer F.Cu) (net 5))
 (segment (start 144.78 96.52) (end 147.32 96.52) (width 0.3048) (layer B.Cu) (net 5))
 (segment (start 147.32 96.52) (end 149.86 96.52) (width 0.3048) (layer B.Cu) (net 5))
 (segment (start 149.86 96.52) (end 152.4 96.52) (width 0.3048) (layer B.Cu) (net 5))
 (segment (start 152.4 96.52) (end 154.94 96.52) (width 0.3048) (layer B.Cu) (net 5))
 (segment (start 154.94 96.52) (end 157.48 96.52) (width 0.3048) (layer B.Cu) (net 5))
 (segment (start 157.48 96.52) (end 160.02 96.52) (width 0.3048) (layer B.Cu) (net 5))
 (segment (start 160.02 96.52) (end 162.56 96.52) (width 0.3048) (layer B.Cu) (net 5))
 (segment (start 147.32 104.14) (end 147.32 101.6) (width 0.3048) (layer B.Cu) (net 5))
 (segment (start 147.32 106.68) (end 147.32 104.14) (width 0.3048) (layer B.Cu) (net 5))
 (segment (start 147.32 107.7595) (end 147.32 106.68) (width 0.3048) (layer B.Cu) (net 5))
 (segment (start 147.32 109.22) (end 147.32 108.1405) (width 0.3048) (layer B.Cu) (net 5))
 (segment (start 154.94 107.95) (end 154.94 107.7595) (width 0.2032) (layer B.Cu) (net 2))
 (segment (start 154.94 107.95) (end 154.94 108.1405) (width 0.2032) (layer B.Cu) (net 2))
 (segment (start 154.94 108.1405) (end 154.94 109.22) (width 0.2032) (layer B.Cu) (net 2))
 (segment (start 154.94 106.68) (end 154.94 104.14) (width 0.3048) (layer B.Cu) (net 2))
 (segment (start 154.94 104.14) (end 154.94 101.6) (width 0.3048) (layer B.Cu) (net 2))
 (segment (start 154.94 107.7595) (end 154.94 106.68) (width 0.3048) (layer B.Cu) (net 2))
 (segment (start 154.94 109.22) (end 154.94 108.1405) (width 0.3048) (layer B.Cu) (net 2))
 (segment (start 152.4 107.7595) (end 152.4 107.95) (width 0.2032) (layer B.Cu) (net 3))
 (segment (start 152.4 107.95) (end 152.4 108.1405) (width 0.2032) (layer B.Cu) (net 3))
 (segment (start 152.4 108.1405) (end 152.4 109.22) (width 0.2032) (layer B.Cu) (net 3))
 (segment (start 152.4 106.68) (end 152.4 104.14) (width 0.3048) (layer B.Cu) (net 3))
 (segment (start 152.4 104.14) (end 152.4 101.6) (width 0.3048) (layer B.Cu) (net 3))
 (segment (start 152.4 109.22) (end 152.4 108.1405) (width 0.3048) (layer B.Cu) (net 3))
 (segment (start 152.4 106.68) (end 152.4 107.7595) (width 0.3048) (layer B.Cu) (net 3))
 (segment (start 149.86 107.7595) (end 149.86 107.95) (width 0.2032) (layer B.Cu) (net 4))
 (segment (start 149.86 107.95) (end 149.86 108.1405) (width 0.2032) (layer B.Cu) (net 4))
 (segment (start 149.86 108.1405) (end 149.86 109.22) (width 0.2032) (layer B.Cu) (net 4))
 (segment (start 149.86 106.68) (end 149.86 104.14) (width 0.3048) (layer B.Cu) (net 4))
 (segment (start 149.86 104.14) (end 149.86 101.6) (width 0.3048) (layer B.Cu) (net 4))
 (segment (start 149.86 107.7595) (end 149.86 106.68) (width 0.3048) (layer B.Cu) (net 4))
 (segment (start 149.86 109.22) (end 149.86 108.1405) (width 0.3048) (layer B.Cu) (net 4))
 (segment (start 154.94 87.8205) (end 154.94 87.63) (width 0.2032) (layer B.Cu) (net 10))
 (segment (start 154.94 87.63) (end 154.94 87.4395) (width 0.2032) (layer B.Cu) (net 10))
 (segment (start 154.94 87.4395) (end 154.94 86.36) (width 0.2032) (layer B.Cu) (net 10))
 (segment (start 154.94 88.9) (end 154.94 91.44) (width 0.3048) (layer B.Cu) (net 10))
 (segment (start 154.94 91.44) (end 154.94 93.98) (width 0.3048) (layer B.Cu) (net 10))
 (segment (start 154.94 86.36) (end 154.94 87.4395) (width 0.3048) (layer B.Cu) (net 10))
 (segment (start 154.94 88.9) (end 154.94 87.8205) (width 0.3048) (layer B.Cu) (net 10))
 (segment (start 152.4 87.8205) (end 152.4 87.63) (width 0.2032) (layer B.Cu) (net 11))
 (segment (start 152.4 87.63) (end 152.4 86.36) (width 0.2032) (layer B.Cu) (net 11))
 (segment (start 152.4 88.9) (end 152.4 91.44) (width 0.3048) (layer B.Cu) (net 11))
 (segment (start 152.4 91.44) (end 152.4 93.98) (width 0.3048) (layer B.Cu) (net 11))
 (segment (start 152.4 88.9) (end 152.4 87.8205) (width 0.3048) (layer B.Cu) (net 11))
 (segment (start 152.4 86.36) (end 152.4 87.4395) (width 0.3048) (layer B.Cu) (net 11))
 (segment (start 149.86 87.8205) (end 149.86 87.63) (width 0.2032) (layer B.Cu) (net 12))
 (segment (start 149.86 87.63) (end 149.86 86.36) (width 0.2032) (layer B.Cu) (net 12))
 (segment (start 149.86 88.9) (end 149.86 91.44) (width 0.3048) (layer B.Cu) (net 12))
 (segment (start 149.86 91.44) (end 149.86 93.98) (width 0.3048) (layer B.Cu) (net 12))
 (segment (start 149.86 88.9) (end 149.86 87.8205) (width 0.3048) (layer B.Cu) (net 12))
 (segment (start 149.86 86.36) (end 149.86 87.4395) (width 0.3048) (layer B.Cu) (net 12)))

